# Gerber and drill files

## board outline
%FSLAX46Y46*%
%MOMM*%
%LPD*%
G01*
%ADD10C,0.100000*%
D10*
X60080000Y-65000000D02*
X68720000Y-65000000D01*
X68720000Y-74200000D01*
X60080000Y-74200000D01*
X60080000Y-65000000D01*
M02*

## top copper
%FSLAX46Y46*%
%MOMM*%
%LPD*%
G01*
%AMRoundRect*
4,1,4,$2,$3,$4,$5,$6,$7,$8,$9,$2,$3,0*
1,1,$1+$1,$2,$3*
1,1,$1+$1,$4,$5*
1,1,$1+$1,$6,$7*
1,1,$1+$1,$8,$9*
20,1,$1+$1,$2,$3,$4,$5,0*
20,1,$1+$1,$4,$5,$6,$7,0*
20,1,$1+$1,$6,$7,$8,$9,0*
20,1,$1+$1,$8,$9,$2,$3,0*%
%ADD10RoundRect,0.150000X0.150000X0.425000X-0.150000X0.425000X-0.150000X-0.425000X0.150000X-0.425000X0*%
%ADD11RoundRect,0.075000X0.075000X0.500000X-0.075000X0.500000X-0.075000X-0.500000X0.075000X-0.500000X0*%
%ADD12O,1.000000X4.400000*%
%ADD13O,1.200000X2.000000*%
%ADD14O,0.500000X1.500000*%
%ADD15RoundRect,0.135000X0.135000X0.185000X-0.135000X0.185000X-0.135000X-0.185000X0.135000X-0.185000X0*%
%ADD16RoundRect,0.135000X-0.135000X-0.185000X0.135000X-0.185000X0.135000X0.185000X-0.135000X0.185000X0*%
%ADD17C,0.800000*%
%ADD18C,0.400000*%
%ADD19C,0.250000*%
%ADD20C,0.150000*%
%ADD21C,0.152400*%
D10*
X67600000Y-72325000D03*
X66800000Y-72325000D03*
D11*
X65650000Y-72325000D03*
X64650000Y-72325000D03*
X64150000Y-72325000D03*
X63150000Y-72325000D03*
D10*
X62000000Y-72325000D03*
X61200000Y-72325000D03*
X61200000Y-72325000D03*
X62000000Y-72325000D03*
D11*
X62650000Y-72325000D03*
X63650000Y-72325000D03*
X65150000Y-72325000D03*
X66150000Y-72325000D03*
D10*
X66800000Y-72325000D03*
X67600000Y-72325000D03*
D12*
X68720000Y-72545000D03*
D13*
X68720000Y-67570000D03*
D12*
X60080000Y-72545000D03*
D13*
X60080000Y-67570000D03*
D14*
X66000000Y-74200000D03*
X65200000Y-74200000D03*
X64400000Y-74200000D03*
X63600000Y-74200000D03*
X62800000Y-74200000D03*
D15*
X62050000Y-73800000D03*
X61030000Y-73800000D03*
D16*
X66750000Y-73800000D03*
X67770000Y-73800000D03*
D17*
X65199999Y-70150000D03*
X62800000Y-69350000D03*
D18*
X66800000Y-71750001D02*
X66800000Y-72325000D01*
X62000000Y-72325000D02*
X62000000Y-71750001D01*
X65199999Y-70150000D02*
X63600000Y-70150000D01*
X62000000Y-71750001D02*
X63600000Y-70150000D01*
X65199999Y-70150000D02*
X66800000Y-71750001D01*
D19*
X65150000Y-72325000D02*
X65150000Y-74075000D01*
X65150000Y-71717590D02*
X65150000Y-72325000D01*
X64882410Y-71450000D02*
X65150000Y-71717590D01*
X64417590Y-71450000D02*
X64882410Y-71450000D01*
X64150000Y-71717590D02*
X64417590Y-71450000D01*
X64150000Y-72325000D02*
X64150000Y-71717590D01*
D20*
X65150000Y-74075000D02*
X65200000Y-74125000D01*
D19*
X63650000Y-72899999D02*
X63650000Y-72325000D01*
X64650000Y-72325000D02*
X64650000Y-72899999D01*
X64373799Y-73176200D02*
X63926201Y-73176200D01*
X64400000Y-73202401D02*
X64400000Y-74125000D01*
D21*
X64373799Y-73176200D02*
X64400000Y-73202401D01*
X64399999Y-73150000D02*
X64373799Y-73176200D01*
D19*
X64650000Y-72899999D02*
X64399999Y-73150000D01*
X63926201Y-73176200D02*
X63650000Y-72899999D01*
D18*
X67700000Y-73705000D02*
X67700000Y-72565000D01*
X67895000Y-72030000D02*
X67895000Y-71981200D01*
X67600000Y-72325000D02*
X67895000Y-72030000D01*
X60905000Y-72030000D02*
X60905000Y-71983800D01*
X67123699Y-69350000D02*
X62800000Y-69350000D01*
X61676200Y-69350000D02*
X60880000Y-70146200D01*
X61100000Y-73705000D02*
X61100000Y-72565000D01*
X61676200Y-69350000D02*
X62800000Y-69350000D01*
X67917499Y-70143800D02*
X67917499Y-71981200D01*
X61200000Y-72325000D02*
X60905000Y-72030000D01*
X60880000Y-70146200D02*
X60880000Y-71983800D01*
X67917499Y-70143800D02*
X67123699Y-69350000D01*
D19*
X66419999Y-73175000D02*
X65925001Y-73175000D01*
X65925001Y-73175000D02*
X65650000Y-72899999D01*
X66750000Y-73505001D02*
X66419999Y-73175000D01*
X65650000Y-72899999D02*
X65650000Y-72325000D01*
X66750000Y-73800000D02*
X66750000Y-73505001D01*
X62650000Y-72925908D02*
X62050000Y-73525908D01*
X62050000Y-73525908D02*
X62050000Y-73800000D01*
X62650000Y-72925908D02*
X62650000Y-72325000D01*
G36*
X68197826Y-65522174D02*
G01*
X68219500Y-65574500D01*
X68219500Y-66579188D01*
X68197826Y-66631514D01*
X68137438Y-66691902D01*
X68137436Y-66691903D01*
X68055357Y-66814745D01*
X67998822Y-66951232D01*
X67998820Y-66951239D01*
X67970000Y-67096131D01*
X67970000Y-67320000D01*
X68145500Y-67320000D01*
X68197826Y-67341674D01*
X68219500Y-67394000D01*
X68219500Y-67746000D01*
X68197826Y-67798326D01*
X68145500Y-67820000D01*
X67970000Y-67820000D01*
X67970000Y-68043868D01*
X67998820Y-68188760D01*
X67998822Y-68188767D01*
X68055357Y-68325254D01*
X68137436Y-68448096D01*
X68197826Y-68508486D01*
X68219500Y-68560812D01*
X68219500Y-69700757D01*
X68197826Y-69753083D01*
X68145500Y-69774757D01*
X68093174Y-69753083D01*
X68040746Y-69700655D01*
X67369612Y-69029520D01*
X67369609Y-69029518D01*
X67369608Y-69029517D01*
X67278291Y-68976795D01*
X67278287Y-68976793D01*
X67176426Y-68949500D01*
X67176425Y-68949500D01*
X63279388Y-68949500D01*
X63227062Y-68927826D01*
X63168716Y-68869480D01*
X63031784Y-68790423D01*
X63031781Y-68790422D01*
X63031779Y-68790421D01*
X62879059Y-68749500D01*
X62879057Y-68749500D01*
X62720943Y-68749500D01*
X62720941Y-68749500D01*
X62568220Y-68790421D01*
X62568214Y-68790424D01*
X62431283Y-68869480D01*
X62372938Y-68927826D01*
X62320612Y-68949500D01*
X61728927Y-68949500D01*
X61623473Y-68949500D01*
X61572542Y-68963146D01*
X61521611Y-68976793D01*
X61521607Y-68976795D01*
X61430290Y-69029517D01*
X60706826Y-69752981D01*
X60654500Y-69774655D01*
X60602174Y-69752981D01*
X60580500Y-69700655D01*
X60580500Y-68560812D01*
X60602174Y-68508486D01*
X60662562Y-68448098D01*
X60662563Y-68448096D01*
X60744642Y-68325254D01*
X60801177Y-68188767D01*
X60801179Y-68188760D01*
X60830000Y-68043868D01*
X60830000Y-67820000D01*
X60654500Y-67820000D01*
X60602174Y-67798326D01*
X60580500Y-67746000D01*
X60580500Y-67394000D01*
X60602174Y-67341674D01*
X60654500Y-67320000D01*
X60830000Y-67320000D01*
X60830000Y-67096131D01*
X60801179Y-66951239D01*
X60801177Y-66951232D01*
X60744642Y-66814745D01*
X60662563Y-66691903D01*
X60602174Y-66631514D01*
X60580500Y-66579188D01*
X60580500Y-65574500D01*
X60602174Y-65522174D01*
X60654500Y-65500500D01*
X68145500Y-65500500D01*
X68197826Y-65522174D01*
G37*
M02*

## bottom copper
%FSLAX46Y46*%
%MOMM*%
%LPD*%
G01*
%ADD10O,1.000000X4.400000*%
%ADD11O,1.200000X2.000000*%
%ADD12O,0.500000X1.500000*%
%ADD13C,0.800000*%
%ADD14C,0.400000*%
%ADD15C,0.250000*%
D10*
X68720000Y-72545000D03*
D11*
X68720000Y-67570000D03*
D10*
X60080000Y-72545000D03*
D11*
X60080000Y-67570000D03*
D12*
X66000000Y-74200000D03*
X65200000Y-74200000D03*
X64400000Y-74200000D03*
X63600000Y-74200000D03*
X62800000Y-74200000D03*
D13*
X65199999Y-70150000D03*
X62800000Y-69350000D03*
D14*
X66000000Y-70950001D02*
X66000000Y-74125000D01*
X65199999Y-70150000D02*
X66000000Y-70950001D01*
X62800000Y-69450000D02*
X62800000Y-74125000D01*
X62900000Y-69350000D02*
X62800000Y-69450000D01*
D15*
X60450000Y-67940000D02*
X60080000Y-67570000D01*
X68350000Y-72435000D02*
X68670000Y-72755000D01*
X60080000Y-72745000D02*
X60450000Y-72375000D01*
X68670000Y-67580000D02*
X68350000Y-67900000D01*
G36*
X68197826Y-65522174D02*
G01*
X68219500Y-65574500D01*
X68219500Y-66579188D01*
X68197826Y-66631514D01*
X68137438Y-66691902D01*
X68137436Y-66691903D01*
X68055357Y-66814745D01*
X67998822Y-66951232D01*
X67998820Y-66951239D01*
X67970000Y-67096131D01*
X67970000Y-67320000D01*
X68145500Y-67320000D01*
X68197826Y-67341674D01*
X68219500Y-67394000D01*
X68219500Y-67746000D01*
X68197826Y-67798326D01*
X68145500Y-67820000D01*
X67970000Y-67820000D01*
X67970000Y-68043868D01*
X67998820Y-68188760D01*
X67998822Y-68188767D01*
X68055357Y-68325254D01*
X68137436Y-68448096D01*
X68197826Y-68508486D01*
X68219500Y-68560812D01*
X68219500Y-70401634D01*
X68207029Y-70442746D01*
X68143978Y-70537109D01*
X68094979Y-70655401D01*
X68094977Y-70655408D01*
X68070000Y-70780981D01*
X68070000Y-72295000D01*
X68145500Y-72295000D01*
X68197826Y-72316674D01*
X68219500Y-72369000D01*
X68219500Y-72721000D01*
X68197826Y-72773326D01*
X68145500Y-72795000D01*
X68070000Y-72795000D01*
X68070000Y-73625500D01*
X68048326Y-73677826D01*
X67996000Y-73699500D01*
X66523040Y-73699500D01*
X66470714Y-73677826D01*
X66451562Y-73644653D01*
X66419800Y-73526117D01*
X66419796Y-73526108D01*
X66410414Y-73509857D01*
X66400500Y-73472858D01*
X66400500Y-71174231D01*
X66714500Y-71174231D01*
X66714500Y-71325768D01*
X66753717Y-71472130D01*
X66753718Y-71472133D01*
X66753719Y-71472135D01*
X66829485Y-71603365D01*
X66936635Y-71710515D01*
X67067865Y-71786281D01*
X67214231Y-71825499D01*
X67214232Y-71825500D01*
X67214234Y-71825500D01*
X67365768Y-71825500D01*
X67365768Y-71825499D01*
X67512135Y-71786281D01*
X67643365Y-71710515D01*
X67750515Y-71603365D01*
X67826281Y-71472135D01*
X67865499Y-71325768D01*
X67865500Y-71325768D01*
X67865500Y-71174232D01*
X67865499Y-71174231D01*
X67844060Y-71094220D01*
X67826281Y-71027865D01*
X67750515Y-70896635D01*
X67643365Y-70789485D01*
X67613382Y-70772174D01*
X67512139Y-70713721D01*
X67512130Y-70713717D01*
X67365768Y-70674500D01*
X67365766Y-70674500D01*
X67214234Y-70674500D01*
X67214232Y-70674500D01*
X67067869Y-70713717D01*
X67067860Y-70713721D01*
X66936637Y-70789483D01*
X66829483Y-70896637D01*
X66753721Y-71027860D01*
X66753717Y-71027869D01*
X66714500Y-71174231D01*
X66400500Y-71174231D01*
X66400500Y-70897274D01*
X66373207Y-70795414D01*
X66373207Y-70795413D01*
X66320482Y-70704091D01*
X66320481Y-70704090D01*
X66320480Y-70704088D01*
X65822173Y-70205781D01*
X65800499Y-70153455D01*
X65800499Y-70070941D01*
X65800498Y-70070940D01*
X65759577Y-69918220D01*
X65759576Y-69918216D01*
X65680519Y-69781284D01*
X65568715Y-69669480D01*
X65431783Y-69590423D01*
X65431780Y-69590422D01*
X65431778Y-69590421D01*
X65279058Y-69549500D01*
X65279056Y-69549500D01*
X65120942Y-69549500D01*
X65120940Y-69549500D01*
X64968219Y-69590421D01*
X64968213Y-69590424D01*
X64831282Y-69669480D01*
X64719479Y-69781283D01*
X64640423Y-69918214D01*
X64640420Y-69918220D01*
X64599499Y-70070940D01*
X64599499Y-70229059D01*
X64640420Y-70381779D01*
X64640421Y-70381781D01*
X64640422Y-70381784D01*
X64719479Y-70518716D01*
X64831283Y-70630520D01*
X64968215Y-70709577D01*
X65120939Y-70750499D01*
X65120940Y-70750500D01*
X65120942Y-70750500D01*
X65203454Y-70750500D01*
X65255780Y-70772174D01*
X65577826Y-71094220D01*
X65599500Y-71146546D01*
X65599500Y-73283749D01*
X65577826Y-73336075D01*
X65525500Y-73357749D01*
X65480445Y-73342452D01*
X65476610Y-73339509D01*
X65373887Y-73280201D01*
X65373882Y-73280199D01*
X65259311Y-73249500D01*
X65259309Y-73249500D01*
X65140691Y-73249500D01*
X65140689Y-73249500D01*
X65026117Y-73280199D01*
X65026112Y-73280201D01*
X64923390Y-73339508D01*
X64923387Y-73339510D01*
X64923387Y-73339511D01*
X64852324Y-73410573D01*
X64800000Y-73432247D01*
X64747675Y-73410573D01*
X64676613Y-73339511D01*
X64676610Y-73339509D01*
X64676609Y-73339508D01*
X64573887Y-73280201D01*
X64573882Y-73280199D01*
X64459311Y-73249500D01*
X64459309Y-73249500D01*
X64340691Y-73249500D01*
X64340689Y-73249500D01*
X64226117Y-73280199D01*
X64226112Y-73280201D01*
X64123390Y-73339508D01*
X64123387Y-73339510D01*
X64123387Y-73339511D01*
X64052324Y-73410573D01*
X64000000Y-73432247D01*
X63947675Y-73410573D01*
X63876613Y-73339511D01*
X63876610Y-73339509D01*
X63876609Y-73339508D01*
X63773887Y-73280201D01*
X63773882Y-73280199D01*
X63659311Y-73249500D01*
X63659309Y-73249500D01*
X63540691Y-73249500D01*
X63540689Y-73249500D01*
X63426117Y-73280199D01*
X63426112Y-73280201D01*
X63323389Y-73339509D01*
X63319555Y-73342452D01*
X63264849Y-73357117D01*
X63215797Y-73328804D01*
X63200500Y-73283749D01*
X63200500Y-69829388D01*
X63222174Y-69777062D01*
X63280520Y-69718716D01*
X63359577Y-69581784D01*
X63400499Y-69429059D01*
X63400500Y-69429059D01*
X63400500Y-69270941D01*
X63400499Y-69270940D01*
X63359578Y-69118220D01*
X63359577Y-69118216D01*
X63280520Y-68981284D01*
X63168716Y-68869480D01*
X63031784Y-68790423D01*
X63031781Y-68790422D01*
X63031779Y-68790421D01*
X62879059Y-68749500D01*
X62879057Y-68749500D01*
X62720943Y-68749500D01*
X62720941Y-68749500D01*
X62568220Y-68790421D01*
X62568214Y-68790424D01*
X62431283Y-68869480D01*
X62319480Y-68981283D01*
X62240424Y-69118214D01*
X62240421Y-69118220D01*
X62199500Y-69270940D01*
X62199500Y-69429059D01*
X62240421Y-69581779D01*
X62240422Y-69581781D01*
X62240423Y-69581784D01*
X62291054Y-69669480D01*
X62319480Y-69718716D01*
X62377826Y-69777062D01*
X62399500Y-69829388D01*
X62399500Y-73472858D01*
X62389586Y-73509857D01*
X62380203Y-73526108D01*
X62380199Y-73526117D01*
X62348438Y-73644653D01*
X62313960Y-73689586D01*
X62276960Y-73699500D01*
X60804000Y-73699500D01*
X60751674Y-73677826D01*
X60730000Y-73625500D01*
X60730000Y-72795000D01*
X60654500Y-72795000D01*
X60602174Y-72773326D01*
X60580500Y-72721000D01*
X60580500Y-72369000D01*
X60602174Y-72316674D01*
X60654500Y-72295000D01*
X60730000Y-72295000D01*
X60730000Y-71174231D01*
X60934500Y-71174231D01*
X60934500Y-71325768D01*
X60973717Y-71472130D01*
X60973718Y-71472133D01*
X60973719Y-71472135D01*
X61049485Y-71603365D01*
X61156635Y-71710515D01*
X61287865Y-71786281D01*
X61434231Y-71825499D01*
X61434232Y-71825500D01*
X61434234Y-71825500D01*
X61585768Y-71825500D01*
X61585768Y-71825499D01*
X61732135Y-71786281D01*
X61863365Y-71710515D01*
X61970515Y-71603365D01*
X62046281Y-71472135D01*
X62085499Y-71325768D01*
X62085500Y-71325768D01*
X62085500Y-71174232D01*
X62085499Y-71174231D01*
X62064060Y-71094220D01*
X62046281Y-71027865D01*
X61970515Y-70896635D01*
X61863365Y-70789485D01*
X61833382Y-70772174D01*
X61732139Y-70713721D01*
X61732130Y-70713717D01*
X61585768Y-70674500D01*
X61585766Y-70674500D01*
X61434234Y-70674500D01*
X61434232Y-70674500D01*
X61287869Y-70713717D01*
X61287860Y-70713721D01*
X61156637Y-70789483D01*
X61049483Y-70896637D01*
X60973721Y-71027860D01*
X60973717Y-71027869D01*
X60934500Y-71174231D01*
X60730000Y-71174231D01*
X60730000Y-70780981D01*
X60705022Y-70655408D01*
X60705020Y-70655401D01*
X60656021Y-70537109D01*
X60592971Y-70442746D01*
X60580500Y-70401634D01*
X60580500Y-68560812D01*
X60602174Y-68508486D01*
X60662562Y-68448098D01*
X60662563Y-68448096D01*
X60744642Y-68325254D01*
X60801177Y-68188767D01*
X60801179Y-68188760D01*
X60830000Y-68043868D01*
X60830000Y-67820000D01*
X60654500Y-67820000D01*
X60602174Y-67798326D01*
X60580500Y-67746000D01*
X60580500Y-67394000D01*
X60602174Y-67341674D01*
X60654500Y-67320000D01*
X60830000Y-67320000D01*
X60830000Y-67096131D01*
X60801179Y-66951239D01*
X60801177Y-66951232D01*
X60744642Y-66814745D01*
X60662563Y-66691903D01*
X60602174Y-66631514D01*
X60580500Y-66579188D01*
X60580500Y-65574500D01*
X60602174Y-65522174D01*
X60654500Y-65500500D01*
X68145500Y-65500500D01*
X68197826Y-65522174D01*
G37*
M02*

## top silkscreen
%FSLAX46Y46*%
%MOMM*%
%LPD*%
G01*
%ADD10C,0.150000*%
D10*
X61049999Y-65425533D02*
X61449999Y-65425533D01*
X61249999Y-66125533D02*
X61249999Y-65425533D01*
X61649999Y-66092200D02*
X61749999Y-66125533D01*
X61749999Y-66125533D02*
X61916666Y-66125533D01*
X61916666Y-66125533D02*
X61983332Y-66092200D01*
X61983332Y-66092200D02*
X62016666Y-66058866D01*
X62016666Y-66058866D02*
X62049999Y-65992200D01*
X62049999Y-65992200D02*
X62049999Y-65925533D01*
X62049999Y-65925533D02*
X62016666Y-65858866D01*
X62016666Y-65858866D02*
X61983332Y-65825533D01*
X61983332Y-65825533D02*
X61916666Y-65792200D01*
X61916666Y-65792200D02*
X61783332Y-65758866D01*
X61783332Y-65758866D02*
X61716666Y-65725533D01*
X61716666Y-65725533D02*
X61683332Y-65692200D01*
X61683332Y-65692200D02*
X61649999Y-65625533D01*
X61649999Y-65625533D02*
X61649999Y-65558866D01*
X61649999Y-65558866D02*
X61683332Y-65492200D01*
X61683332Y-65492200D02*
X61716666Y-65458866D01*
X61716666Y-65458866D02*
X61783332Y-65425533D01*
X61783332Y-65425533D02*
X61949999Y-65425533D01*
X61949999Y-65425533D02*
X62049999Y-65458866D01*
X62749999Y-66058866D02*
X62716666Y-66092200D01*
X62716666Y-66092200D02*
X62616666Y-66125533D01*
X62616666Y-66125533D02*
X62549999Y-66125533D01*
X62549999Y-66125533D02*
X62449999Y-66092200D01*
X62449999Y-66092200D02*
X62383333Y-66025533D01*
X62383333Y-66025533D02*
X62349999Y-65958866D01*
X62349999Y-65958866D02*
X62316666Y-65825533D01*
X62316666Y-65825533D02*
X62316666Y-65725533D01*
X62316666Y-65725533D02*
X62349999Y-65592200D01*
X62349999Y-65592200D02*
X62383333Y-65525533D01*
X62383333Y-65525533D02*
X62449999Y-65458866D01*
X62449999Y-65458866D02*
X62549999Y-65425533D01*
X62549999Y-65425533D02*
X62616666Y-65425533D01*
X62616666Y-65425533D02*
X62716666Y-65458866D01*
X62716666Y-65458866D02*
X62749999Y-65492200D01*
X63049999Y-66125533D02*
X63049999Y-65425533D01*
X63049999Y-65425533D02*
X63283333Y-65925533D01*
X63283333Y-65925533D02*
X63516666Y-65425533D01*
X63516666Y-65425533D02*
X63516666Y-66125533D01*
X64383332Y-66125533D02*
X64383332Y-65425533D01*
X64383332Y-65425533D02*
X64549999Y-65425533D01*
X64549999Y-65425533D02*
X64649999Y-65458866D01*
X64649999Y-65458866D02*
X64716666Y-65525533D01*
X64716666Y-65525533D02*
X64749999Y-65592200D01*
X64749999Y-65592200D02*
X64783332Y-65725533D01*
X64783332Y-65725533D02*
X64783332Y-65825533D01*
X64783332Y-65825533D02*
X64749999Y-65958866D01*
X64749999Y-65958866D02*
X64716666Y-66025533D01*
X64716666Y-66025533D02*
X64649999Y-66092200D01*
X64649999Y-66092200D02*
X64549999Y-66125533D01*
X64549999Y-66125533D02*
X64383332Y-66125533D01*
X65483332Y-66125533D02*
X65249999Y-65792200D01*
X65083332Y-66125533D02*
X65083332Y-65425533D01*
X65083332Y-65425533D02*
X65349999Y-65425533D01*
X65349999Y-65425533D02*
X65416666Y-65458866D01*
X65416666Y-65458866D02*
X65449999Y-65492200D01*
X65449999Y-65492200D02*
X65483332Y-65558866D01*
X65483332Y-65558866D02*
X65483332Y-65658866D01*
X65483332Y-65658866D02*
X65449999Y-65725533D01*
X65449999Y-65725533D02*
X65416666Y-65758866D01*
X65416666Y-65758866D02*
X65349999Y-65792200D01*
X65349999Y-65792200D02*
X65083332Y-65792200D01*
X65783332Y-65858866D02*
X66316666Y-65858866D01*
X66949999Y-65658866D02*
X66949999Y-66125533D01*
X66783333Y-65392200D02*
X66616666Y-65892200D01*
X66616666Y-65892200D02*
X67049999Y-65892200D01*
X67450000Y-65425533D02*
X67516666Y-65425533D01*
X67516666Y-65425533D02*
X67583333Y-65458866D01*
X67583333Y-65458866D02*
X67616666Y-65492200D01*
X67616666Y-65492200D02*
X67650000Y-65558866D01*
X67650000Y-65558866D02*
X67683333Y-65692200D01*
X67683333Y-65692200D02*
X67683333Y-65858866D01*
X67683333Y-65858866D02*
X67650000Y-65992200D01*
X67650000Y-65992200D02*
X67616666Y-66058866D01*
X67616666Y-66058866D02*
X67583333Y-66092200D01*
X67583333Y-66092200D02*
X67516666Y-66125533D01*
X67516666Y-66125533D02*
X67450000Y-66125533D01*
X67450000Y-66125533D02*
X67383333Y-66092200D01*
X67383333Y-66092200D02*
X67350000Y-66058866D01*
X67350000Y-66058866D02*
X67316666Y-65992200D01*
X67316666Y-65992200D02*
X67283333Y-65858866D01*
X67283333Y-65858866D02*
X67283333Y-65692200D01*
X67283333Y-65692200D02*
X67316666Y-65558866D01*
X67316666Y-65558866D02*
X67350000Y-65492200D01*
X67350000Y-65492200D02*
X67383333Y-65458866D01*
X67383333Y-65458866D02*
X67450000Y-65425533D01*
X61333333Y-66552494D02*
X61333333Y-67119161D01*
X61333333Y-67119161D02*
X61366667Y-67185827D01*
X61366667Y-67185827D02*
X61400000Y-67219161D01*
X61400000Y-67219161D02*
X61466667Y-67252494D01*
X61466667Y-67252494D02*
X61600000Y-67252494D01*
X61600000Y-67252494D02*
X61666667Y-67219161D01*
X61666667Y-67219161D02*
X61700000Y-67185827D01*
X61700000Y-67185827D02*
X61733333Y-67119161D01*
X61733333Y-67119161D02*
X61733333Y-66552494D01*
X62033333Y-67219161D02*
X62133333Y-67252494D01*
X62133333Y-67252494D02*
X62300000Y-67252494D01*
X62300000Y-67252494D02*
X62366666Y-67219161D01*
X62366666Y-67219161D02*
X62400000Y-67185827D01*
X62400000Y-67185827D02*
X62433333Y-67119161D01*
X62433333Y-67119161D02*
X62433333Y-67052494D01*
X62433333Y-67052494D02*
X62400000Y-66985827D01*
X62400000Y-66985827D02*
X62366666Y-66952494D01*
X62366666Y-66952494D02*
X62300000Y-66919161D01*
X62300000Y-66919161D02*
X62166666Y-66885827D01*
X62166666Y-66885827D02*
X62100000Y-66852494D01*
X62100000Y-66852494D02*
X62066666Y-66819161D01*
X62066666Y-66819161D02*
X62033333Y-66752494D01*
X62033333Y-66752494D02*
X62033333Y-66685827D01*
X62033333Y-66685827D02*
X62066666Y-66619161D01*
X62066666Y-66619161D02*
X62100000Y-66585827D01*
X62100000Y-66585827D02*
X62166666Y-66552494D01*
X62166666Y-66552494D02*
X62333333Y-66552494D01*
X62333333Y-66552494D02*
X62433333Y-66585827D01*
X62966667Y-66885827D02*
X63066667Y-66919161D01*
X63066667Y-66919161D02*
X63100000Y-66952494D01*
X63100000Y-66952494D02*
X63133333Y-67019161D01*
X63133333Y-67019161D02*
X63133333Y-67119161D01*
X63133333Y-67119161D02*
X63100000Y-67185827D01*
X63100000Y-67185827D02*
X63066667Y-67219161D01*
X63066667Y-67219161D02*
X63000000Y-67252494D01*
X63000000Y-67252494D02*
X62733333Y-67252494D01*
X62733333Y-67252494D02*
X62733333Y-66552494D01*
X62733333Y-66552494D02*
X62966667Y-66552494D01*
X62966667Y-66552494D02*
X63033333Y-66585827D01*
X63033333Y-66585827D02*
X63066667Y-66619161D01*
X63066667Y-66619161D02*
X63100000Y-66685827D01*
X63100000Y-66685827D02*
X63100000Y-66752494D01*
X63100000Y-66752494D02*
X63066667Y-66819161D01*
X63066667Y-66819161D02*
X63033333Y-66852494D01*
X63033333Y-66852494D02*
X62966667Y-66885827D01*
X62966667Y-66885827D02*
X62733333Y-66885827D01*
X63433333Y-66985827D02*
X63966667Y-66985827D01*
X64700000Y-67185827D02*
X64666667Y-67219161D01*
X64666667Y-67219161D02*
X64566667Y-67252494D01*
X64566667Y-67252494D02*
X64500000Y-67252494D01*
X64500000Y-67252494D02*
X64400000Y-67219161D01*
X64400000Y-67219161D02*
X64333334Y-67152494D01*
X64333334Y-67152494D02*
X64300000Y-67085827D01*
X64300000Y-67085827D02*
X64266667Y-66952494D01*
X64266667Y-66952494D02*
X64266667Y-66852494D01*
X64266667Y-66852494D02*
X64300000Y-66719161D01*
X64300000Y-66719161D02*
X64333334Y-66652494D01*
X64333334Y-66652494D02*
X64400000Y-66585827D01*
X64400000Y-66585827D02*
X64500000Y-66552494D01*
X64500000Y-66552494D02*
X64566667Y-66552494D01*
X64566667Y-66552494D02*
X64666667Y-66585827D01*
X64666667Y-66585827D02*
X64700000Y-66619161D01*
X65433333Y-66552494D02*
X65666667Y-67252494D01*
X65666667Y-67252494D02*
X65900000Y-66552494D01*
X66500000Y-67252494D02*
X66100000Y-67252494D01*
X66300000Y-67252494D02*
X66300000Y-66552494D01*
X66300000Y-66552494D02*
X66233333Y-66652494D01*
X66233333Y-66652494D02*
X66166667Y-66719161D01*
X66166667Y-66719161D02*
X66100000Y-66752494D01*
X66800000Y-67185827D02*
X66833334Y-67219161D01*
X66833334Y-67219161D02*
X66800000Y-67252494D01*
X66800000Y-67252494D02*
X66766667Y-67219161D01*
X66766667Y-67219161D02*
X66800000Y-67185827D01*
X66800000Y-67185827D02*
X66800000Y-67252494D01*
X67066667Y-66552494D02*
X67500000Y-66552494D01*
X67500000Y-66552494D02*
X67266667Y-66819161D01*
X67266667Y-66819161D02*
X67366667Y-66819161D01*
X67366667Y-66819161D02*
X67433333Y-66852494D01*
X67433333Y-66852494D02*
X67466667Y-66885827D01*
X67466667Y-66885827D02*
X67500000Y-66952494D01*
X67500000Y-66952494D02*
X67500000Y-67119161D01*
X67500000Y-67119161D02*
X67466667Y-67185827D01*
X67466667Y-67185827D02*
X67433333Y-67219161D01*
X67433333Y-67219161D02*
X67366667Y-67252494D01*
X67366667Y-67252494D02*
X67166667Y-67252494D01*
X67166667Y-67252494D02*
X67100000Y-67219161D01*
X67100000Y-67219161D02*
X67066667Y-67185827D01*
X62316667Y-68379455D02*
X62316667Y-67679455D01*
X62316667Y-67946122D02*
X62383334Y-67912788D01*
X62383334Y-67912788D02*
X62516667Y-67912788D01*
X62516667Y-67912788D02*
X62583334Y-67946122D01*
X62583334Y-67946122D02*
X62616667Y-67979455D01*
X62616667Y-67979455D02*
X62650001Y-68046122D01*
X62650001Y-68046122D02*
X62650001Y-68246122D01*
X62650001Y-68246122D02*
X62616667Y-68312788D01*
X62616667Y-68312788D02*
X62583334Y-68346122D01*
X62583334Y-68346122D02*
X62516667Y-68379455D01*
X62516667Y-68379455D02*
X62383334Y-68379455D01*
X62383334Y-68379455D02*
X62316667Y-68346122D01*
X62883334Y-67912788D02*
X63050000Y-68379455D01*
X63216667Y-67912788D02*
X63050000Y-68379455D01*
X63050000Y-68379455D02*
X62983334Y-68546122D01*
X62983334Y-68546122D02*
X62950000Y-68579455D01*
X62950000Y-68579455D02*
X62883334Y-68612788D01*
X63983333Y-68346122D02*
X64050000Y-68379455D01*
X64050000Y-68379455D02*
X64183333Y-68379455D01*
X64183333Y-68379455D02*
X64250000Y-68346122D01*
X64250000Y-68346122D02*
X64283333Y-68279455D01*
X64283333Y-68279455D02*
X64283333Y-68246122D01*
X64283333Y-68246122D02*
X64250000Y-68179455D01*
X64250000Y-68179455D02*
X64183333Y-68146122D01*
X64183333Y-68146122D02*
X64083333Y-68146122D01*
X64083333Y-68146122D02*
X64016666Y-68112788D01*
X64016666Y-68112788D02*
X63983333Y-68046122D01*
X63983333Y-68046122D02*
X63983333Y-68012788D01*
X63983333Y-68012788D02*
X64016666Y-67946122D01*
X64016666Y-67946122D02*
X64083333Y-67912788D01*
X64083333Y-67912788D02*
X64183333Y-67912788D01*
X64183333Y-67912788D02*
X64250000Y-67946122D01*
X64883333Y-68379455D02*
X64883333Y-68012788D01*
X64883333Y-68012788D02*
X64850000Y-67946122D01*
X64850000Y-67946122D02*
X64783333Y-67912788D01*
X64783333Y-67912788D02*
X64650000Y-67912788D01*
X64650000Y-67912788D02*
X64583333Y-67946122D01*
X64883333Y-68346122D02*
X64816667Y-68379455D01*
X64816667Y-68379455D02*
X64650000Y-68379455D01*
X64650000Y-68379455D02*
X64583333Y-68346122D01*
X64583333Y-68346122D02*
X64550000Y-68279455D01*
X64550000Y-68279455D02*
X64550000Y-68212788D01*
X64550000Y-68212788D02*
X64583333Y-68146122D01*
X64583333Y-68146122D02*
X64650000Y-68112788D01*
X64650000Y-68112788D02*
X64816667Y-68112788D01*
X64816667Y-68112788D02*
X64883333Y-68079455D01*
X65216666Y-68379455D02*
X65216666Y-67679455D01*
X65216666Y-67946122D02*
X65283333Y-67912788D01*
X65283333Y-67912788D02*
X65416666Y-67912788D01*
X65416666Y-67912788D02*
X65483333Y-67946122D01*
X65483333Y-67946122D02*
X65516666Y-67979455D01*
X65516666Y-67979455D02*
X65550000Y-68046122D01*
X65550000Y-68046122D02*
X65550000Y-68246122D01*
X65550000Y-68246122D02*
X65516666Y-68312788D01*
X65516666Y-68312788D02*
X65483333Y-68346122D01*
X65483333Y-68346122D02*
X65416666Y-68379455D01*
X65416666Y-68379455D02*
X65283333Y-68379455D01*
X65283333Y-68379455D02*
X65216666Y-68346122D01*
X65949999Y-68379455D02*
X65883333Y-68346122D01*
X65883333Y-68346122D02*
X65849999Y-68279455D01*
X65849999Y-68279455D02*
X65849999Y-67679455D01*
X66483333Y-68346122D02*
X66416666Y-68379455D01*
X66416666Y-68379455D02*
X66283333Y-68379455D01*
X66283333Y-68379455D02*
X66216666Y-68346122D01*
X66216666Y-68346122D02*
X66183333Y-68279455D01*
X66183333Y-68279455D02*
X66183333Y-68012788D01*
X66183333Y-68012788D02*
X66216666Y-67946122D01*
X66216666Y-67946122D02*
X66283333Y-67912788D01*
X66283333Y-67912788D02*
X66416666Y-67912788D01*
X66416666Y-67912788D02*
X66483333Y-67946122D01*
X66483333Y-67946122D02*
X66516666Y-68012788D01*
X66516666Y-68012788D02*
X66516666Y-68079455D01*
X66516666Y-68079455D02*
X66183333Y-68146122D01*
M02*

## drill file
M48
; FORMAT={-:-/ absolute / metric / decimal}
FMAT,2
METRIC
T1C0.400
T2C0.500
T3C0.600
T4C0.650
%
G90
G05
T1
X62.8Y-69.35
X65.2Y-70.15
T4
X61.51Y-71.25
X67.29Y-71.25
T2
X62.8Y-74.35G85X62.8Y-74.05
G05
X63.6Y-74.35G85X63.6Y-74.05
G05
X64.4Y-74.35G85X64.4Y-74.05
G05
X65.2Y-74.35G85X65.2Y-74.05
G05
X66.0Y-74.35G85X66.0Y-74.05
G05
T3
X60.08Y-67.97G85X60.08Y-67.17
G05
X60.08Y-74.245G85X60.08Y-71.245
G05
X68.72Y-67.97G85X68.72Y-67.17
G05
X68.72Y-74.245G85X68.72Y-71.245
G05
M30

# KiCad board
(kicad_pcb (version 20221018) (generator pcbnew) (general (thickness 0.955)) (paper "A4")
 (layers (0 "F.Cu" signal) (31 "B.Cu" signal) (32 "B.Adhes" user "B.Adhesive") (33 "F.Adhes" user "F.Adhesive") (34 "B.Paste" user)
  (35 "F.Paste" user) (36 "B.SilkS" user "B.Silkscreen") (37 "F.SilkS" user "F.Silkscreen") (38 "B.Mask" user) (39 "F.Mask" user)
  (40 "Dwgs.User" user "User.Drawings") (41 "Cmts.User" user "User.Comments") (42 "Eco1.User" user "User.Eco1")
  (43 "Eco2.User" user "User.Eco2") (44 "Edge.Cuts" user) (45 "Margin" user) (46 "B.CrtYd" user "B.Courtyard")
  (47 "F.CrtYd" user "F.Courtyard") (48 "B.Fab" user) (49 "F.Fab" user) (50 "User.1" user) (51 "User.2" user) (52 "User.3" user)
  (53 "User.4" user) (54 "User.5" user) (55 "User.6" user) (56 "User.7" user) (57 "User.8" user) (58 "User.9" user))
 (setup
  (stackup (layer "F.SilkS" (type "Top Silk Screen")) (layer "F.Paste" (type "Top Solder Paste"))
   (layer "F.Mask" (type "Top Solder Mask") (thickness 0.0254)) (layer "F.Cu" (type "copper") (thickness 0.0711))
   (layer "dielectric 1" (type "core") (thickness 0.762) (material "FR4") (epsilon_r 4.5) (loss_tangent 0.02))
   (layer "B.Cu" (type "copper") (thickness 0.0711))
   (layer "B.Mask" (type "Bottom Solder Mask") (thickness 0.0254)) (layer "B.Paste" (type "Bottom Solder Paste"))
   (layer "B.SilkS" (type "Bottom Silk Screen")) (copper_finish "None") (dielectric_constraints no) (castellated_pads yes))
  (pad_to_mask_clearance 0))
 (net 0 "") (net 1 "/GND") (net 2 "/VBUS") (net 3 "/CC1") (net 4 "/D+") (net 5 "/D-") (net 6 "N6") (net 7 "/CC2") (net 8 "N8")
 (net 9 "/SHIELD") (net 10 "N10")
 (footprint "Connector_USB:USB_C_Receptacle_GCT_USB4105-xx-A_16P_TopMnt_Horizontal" (layer "F.Cu") (at 64.4 68.645 180)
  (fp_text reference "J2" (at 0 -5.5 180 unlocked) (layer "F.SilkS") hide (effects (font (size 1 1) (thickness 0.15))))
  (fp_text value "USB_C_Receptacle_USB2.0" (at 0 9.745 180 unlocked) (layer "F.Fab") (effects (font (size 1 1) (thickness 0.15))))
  (pad "" np_thru_hole circle (at -2.89 -2.605 180) (size 0.65 0.65) (drill 0.65) (layers "F&B.Cu" "*.Mask"))
  (pad "" np_thru_hole circle (at 2.89 -2.605 180) (size 0.65 0.65) (drill 0.65) (layers "F&B.Cu" "*.Mask"))
  (pad "A1" smd roundrect (at -3.2 -3.68 180) (size 0.6 1.15) (layers "F.Cu" "F.Paste" "F.Mask") (roundrect_rratio 0.25) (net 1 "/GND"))
  (pad "A4" smd roundrect (at -2.4 -3.68 180) (size 0.6 1.15) (layers "F.Cu" "F.Paste" "F.Mask") (roundrect_rratio 0.25) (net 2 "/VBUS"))
  (pad "A5" smd roundrect (at -1.25 -3.68 180) (size 0.3 1.15) (layers "F.Cu" "F.Paste" "F.Mask") (roundrect_rratio 0.25) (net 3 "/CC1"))
  (pad "A6" smd roundrect (at -0.25 -3.68 180) (size 0.3 1.15) (layers "F.Cu" "F.Paste" "F.Mask") (roundrect_rratio 0.25) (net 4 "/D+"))
  (pad "A7" smd roundrect (at 0.25 -3.68 180) (size 0.3 1.15) (layers "F.Cu" "F.Paste" "F.Mask") (roundrect_rratio 0.25) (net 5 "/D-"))
  (pad "A8" smd roundrect (at 1.25 -3.68 180) (size 0.3 1.15) (layers "F.Cu" "F.Paste" "F.Mask") (roundrect_rratio 0.25) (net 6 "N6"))
  (pad "A9" smd roundrect (at 2.4 -3.68 180) (size 0.6 1.15) (layers "F.Cu" "F.Paste" "F.Mask") (roundrect_rratio 0.25) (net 2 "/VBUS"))
  (pad "A12" smd roundrect (at 3.2 -3.68 180) (size 0.6 1.15) (layers "F.Cu" "F.Paste" "F.Mask") (roundrect_rratio 0.25) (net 1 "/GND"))
  (pad "B1" smd roundrect (at 3.2 -3.68 180) (size 0.6 1.15) (layers "F.Cu" "F.Paste" "F.Mask") (roundrect_rratio 0.25) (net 1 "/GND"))
  (pad "B4" smd roundrect (at 2.4 -3.68 180) (size 0.6 1.15) (layers "F.Cu" "F.Paste" "F.Mask") (roundrect_rratio 0.25) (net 2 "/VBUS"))
  (pad "B5" smd roundrect (at 1.75 -3.68 180) (size 0.3 1.15) (layers "F.Cu" "F.Paste" "F.Mask") (roundrect_rratio 0.25) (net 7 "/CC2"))
  (pad "B6" smd roundrect (at 0.75 -3.68 180) (size 0.3 1.15) (layers "F.Cu" "F.Paste" "F.Mask") (roundrect_rratio 0.25) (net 4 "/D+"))
  (pad "B7" smd roundrect (at -0.75 -3.68 180) (size 0.3 1.15) (layers "F.Cu" "F.Paste" "F.Mask") (roundrect_rratio 0.25) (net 5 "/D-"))
  (pad "B8" smd roundrect (at -1.75 -3.68 180) (size 0.3 1.15) (layers "F.Cu" "F.Paste" "F.Mask") (roundrect_rratio 0.25) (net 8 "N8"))
  (pad "B9" smd roundrect (at -2.4 -3.68 180) (size 0.6 1.15) (layers "F.Cu" "F.Paste" "F.Mask") (roundrect_rratio 0.25) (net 2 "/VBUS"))
  (pad "B12" smd roundrect (at -3.2 -3.68 180) (size 0.6 1.15) (layers "F.Cu" "F.Paste" "F.Mask") (roundrect_rratio 0.25) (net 1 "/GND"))
  (pad "S1" thru_hole oval (at -4.32 -4.1 180) (size 1 4.4) (drill oval 0.6 3.6 (offset 0 0.2)) (layers "*.Cu" "*.Mask" "F.Paste")
   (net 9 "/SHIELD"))
  (pad "S1" thru_hole oval (at -4.32 1.075 180) (size 1.2 2) (drill oval 0.6 1.4) (layers "*.Cu" "*.Mask" "F.Paste") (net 9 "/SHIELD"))
  (pad "S1" thru_hole oval (at 4.32 -4.1 180) (size 1 4.4) (drill oval 0.6 3.6 (offset 0 0.2)) (layers "*.Cu" "*.Mask" "F.Paste")
   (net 9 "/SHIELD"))
  (pad "S1" thru_hole oval (at 4.32 1.075 180) (size 1.2 2) (drill oval 0.6 1.4) (layers "*.Cu" "*.Mask" "F.Paste") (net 9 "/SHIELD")))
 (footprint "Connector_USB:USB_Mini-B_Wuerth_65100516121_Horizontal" (layer "F.Cu") (at 64.4 72.35 180)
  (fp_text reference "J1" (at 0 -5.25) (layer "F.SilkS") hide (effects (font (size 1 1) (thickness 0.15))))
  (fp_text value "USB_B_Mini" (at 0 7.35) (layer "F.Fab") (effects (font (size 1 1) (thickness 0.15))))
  (pad "1" thru_hole oval (at -1.6 -1.85 180) (size 0.5 1.5) (drill oval 0.5 0.8) (layers "*.Cu" "*.Mask") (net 2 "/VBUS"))
  (pad "2" thru_hole oval (at -0.8 -1.85 180) (size 0.5 1.5) (drill oval 0.5 0.8) (layers "*.Cu" "*.Mask") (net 5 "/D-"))
  (pad "3" thru_hole oval (at 0 -1.85 180) (size 0.5 1.5) (drill oval 0.5 0.8) (layers "*.Cu" "*.Mask") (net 4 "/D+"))
  (pad "4" thru_hole oval (at 0.8 -1.85 180) (size 0.5 1.5) (drill oval 0.5 0.8) (layers "*.Cu" "*.Mask") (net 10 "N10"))
  (pad "5" thru_hole oval (at 1.6 -1.85 180) (size 0.5 1.5) (drill oval 0.5 0.8) (layers "*.Cu" "*.Mask") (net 1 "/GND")))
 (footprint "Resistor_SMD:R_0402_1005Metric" (layer "F.Cu") (at 61.54 73.8 180)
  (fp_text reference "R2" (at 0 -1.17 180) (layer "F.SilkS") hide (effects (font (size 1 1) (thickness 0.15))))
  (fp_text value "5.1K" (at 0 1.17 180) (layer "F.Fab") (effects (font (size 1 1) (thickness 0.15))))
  (pad "1" smd roundrect (at -0.51 0 180) (size 0.54 0.64) (layers "F.Cu" "F.Paste" "F.Mask") (roundrect_rratio 0.25) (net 7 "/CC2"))
  (pad "2" smd roundrect (at 0.51 0 180) (size 0.54 0.64) (layers "F.Cu" "F.Paste" "F.Mask") (roundrect_rratio 0.25) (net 1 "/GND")))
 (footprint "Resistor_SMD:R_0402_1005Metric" (layer "F.Cu") (at 67.26 73.8)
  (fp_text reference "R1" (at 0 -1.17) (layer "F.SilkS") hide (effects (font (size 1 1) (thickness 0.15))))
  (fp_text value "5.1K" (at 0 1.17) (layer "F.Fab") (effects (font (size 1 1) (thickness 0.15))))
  (pad "1" smd roundrect (at -0.51 0) (size 0.54 0.64) (layers "F.Cu" "F.Paste" "F.Mask") (roundrect_rratio 0.25) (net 3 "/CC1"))
  (pad "2" smd roundrect (at 0.51 0) (size 0.54 0.64) (layers "F.Cu" "F.Paste" "F.Mask") (roundrect_rratio 0.25) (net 1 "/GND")))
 (gr_rect locked (start 60.08 65) (end 68.72 74.2) (stroke (width 0.1) (type default)) (fill none) (layer "Edge.Cuts"))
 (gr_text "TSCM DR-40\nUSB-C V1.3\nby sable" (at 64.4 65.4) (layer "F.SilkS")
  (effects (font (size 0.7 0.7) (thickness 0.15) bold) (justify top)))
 (segment (start 66.8 71.750001) (end 66.8 72.325) (width 0.4) (layer "F.Cu") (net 2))
 (segment (start 62 72.325) (end 62 71.750001) (width 0.4) (layer "F.Cu") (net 2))
 (segment (start 65.199999 70.15) (end 63.6 70.15) (width 0.4) (layer "F.Cu") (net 2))
 (segment (start 62 71.750001) (end 63.6 70.15) (width 0.4) (layer "F.Cu") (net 2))
 (segment (start 65.199999 70.15) (end 66.8 71.750001) (width 0.4) (layer "F.Cu") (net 2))
 (via (at 65.199999 70.15) (size 0.8) (drill 0.4) (layers "F.Cu" "B.Cu") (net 2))
 (segment (start 66 70.950001) (end 66 74.125) (width 0.4) (layer "B.Cu") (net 2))
 (segment (start 65.199999 70.15) (end 66 70.950001) (width 0.4) (layer "B.Cu") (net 2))
 (segment (start 65.15 72.325) (end 65.15 74.075) (width 0.25) (layer "F.Cu") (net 5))
 (segment (start 65.15 71.71759) (end 65.15 72.325) (width 0.25) (layer "F.Cu") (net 5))
 (segment (start 64.88241 71.45) (end 65.15 71.71759) (width 0.25) (layer "F.Cu") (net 5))
 (segment (start 64.41759 71.45) (end 64.88241 71.45) (width 0.25) (layer "F.Cu") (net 5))
 (segment (start 64.15 71.71759) (end 64.41759 71.45) (width 0.25) (layer "F.Cu") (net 5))
 (segment (start 64.15 72.325) (end 64.15 71.71759) (width 0.25) (layer "F.Cu") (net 5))
 (segment (start 65.15 74.075) (end 65.2 74.125) (width 0.15) (layer "F.Cu") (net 5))
 (segment (start 63.65 72.899999) (end 63.65 72.325) (width 0.25) (layer "F.Cu") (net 4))
 (segment (start 64.65 72.325) (end 64.65 72.899999) (width 0.25) (layer "F.Cu") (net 4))
 (segment (start 64.373799 73.1762) (end 63.926201 73.1762) (width 0.25) (layer "F.Cu") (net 4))
 (segment (start 64.4 73.202401) (end 64.4 74.125) (width 0.25) (layer "F.Cu") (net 4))
 (segment (start 64.373799 73.1762) (end 64.4 73.202401) (width 0.1524) (layer "F.Cu") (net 4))
 (segment (start 64.399999 73.15) (end 64.373799 73.1762) (width 0.1524) (layer "F.Cu") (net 4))
 (segment (start 64.65 72.899999) (end 64.399999 73.15) (width 0.25) (layer "F.Cu") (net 4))
 (segment (start 63.926201 73.1762) (end 63.65 72.899999) (width 0.25) (layer "F.Cu") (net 4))
 (segment (start 67.7 73.705) (end 67.7 72.565) (width 0.4) (layer "F.Cu") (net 1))
 (segment (start 67.895 72.03) (end 67.895 71.9812) (width 0.4) (layer "F.Cu") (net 1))
 (segment (start 67.6 72.325) (end 67.895 72.03) (width 0.4) (layer "F.Cu") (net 1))
 (segment (start 60.905 72.03) (end 60.905 71.9838) (width 0.4) (layer "F.Cu") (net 1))
 (segment (start 67.123699 69.35) (end 62.8 69.35) (width 0.4) (layer "F.Cu") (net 1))
 (segment (start 61.6762 69.35) (end 60.88 70.1462) (width 0.4) (layer "F.Cu") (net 1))
 (segment (start 61.1 73.705) (end 61.1 72.565) (width 0.4) (layer "F.Cu") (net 1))
 (segment (start 61.6762 69.35) (end 62.8 69.35) (width 0.4) (layer "F.Cu") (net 1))
 (segment (start 67.917499 70.1438) (end 67.917499 71.9812) (width 0.4) (layer "F.Cu") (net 1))
 (segment (start 61.2 72.325) (end 60.905 72.03) (width 0.4) (layer "F.Cu") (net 1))
 (segment (start 60.88 70.1462) (end 60.88 71.9838) (width 0.4) (layer "F.Cu") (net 1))
 (segment (start 67.917499 70.1438) (end 67.123699 69.35) (width 0.4) (layer "F.Cu") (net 1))
 (via (at 62.8 69.35) (size 0.8) (drill 0.4) (layers "F.Cu" "B.Cu") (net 1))
 (segment (start 62.8 69.45) (end 62.8 74.125) (width 0.4) (layer "B.Cu") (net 1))
 (segment (start 62.9 69.35) (end 62.8 69.45) (width 0.4) (layer "B.Cu") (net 1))
 (segment (start 66.419999 73.175) (end 65.925001 73.175) (width 0.25) (layer "F.Cu") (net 3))
 (segment (start 65.925001 73.175) (end 65.65 72.899999) (width 0.25) (layer "F.Cu") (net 3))
 (segment (start 66.75 73.505001) (end 66.419999 73.175) (width 0.25) (layer "F.Cu") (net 3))
 (segment (start 65.65 72.899999) (end 65.65 72.325) (width 0.25) (layer "F.Cu") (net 3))
 (segment (start 66.75 73.8) (end 66.75 73.505001) (width 0.25) (layer "F.Cu") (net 3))
 (segment (start 62.65 72.925908) (end 62.05 73.525908) (width 0.25) (layer "F.Cu") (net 7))
 (segment (start 62.05 73.525908) (end 62.05 73.8) (width 0.25) (layer "F.Cu") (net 7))
 (segment (start 62.65 72.925908) (end 62.65 72.325) (width 0.25) (layer "F.Cu") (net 7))
 (segment (start 60.45 67.94) (end 60.08 67.57) (width 0.25) (layer "B.Cu") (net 9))
 (segment (start 68.35 72.435) (end 68.67 72.755) (width 0.25) (layer "B.Cu") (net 9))
 (segment (start 60.08 72.745) (end 60.45 72.375) (width 0.25) (layer "B.Cu") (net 9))
 (segment (start 68.67 67.58) (end 68.35 67.9) (width 0.25) (layer "B.Cu") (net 9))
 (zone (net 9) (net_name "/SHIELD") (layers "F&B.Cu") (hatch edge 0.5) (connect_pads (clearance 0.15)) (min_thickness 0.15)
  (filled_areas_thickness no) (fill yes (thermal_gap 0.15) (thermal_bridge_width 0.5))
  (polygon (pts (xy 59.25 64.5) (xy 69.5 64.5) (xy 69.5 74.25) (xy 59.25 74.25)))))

